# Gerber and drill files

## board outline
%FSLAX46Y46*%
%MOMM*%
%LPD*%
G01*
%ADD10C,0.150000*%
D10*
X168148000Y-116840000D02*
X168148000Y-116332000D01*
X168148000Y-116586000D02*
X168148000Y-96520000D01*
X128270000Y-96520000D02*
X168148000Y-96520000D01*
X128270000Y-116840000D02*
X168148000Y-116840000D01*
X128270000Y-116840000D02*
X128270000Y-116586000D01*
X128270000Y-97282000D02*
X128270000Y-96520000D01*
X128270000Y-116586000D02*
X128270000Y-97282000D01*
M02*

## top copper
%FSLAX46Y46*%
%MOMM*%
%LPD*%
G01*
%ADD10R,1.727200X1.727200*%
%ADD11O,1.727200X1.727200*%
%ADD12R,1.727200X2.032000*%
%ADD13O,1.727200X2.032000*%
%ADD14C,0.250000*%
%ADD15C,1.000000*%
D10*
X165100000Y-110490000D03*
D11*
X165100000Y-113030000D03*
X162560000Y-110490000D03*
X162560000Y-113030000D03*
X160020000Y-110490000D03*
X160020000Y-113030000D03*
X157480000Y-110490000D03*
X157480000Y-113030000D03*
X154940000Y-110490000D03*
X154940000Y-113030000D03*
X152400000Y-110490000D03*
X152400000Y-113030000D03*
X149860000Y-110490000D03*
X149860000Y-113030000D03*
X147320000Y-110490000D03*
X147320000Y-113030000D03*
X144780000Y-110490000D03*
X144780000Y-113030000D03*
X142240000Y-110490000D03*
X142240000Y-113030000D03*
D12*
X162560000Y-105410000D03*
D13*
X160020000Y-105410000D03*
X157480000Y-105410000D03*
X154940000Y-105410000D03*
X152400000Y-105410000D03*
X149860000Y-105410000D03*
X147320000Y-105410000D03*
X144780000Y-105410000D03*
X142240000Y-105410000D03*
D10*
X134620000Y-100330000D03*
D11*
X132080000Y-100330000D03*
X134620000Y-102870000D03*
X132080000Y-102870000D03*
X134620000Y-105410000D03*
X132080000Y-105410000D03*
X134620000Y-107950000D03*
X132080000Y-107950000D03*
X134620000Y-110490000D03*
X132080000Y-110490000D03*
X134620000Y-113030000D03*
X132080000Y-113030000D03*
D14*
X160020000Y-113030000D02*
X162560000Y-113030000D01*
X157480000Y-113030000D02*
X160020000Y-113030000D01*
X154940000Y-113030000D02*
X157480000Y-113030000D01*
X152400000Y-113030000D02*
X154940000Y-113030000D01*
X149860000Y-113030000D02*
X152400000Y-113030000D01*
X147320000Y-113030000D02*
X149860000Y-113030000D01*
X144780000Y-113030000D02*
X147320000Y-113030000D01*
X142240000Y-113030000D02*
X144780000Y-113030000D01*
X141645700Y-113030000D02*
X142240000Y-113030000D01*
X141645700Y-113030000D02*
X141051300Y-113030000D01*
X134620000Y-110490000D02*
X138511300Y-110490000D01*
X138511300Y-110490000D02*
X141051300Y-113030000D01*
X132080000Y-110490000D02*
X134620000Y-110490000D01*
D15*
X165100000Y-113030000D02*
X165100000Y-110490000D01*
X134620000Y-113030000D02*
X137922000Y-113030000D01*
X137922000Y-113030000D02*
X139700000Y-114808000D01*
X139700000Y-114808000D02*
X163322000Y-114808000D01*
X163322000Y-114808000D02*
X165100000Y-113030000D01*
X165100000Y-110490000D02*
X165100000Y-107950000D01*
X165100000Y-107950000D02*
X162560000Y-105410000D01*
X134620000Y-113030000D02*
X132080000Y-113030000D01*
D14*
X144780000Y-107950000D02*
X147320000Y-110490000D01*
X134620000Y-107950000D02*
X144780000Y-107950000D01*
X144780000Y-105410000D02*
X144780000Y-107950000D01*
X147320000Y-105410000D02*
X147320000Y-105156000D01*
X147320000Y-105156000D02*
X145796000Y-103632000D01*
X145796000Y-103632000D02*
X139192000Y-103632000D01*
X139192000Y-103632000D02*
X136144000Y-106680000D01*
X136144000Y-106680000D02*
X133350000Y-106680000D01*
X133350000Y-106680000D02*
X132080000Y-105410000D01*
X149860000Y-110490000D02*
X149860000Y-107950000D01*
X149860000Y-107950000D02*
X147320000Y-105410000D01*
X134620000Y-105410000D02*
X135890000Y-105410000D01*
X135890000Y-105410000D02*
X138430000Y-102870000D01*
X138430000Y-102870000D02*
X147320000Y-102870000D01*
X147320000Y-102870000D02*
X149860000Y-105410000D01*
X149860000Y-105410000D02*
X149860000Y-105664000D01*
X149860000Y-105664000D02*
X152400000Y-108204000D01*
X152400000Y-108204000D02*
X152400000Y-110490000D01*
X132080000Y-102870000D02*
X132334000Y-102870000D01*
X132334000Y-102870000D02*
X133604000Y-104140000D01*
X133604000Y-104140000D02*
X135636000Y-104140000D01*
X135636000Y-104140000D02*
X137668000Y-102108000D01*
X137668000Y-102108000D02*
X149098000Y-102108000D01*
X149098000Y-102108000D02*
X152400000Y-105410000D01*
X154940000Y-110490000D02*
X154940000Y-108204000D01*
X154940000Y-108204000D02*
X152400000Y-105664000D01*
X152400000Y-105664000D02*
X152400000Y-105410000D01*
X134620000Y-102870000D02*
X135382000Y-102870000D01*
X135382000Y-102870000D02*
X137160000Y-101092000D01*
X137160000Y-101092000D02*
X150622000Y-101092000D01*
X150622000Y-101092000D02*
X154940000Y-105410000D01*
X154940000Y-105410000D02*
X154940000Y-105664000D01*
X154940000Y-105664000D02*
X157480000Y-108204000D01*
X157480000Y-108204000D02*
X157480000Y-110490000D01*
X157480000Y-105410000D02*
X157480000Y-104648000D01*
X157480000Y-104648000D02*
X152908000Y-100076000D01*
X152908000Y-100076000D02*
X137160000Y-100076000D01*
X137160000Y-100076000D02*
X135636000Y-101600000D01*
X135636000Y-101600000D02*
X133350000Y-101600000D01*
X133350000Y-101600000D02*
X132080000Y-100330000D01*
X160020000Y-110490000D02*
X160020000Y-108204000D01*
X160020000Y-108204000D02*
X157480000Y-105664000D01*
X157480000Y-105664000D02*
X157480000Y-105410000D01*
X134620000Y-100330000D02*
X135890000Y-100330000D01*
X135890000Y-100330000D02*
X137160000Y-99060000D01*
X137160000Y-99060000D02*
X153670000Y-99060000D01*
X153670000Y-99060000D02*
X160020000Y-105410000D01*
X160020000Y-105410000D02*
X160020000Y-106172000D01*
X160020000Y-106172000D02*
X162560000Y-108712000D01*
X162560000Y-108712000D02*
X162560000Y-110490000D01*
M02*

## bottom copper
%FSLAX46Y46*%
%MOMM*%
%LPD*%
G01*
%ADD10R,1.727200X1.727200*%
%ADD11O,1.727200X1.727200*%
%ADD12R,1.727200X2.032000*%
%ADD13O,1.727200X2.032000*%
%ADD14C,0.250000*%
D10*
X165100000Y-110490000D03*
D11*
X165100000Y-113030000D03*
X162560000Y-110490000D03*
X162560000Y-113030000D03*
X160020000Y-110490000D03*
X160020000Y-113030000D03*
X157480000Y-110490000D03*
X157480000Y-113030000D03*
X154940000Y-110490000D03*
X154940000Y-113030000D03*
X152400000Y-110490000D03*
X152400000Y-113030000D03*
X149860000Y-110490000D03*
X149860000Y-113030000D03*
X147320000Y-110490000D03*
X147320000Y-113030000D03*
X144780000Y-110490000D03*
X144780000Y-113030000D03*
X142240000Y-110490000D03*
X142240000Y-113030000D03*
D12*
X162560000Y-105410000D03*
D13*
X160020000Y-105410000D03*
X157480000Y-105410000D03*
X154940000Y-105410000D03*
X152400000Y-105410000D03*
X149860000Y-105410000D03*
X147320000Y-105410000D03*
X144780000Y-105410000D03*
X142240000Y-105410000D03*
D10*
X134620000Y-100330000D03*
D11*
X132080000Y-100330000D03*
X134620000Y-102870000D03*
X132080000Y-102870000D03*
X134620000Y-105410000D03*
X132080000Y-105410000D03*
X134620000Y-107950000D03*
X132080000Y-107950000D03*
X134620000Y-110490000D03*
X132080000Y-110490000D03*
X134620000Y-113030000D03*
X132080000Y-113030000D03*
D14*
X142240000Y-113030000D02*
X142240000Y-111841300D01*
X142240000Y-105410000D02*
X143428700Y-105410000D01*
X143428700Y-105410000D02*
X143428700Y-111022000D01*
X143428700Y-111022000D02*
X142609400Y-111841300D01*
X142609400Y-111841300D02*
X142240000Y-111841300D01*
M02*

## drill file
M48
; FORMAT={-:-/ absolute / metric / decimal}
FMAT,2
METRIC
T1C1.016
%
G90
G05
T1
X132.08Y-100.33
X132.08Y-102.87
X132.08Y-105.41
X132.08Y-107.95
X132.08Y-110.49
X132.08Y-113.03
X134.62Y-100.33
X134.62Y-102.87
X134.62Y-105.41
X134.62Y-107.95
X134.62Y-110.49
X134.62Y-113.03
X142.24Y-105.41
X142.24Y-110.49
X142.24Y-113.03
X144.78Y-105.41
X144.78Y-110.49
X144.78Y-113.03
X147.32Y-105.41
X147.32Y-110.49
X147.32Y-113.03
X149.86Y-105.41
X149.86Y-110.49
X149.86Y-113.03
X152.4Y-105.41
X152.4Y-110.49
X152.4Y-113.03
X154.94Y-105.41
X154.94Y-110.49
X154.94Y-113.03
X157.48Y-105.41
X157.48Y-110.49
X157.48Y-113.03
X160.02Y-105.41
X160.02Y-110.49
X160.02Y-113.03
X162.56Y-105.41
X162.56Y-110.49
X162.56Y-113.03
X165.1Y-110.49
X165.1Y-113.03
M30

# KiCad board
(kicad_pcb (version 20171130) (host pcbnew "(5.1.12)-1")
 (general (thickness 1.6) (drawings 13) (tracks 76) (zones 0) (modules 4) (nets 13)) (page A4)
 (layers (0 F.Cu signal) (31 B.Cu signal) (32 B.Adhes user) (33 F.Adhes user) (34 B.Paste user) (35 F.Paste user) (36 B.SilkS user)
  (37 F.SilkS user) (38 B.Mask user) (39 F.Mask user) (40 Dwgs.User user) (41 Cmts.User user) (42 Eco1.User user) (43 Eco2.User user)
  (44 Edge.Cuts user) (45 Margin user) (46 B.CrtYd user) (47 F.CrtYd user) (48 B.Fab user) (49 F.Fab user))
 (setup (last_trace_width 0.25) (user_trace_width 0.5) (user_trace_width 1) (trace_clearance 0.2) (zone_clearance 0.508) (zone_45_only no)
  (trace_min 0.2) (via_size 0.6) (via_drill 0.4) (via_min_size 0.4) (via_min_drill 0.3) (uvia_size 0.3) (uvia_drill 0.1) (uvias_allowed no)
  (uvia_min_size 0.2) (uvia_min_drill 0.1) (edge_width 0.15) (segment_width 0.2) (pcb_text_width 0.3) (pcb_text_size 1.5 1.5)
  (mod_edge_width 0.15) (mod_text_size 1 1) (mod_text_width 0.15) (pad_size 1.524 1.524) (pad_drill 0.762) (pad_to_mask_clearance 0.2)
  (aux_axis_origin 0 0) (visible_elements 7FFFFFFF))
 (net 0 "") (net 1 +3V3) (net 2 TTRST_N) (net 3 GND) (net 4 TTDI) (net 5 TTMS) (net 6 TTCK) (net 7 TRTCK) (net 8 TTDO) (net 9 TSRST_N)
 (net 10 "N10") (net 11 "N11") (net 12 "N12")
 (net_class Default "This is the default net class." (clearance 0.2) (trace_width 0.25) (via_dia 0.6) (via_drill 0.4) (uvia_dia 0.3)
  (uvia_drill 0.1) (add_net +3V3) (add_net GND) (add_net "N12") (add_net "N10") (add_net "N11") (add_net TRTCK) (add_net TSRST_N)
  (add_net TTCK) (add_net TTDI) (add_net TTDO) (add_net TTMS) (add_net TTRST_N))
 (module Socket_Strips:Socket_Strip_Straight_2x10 (layer B.Cu) (at 165.1 110.49 180)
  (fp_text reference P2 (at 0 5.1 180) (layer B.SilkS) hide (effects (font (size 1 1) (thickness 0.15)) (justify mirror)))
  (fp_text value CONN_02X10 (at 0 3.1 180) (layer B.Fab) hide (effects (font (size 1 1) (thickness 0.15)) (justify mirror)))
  (pad 1 thru_hole rect (at 0 0 180) (size 1.7272 1.7272) (drill 1.016) (layers *.Cu *.Mask B.SilkS) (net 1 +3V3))
  (pad 2 thru_hole oval (at 0 -2.54 180) (size 1.7272 1.7272) (drill 1.016) (layers *.Cu *.Mask B.SilkS) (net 1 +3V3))
  (pad 3 thru_hole oval (at 2.54 0 180) (size 1.7272 1.7272) (drill 1.016) (layers *.Cu *.Mask B.SilkS) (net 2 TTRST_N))
  (pad 4 thru_hole oval (at 2.54 -2.54 180) (size 1.7272 1.7272) (drill 1.016) (layers *.Cu *.Mask B.SilkS) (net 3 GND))
  (pad 5 thru_hole oval (at 5.08 0 180) (size 1.7272 1.7272) (drill 1.016) (layers *.Cu *.Mask B.SilkS) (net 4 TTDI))
  (pad 6 thru_hole oval (at 5.08 -2.54 180) (size 1.7272 1.7272) (drill 1.016) (layers *.Cu *.Mask B.SilkS) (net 3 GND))
  (pad 7 thru_hole oval (at 7.62 0 180) (size 1.7272 1.7272) (drill 1.016) (layers *.Cu *.Mask B.SilkS) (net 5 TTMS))
  (pad 8 thru_hole oval (at 7.62 -2.54 180) (size 1.7272 1.7272) (drill 1.016) (layers *.Cu *.Mask B.SilkS) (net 3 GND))
  (pad 9 thru_hole oval (at 10.16 0 180) (size 1.7272 1.7272) (drill 1.016) (layers *.Cu *.Mask B.SilkS) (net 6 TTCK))
  (pad 10 thru_hole oval (at 10.16 -2.54 180) (size 1.7272 1.7272) (drill 1.016) (layers *.Cu *.Mask B.SilkS) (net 3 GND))
  (pad 11 thru_hole oval (at 12.7 0 180) (size 1.7272 1.7272) (drill 1.016) (layers *.Cu *.Mask B.SilkS) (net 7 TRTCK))
  (pad 12 thru_hole oval (at 12.7 -2.54 180) (size 1.7272 1.7272) (drill 1.016) (layers *.Cu *.Mask B.SilkS) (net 3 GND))
  (pad 13 thru_hole oval (at 15.24 0 180) (size 1.7272 1.7272) (drill 1.016) (layers *.Cu *.Mask B.SilkS) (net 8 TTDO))
  (pad 14 thru_hole oval (at 15.24 -2.54 180) (size 1.7272 1.7272) (drill 1.016) (layers *.Cu *.Mask B.SilkS) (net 3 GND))
  (pad 15 thru_hole oval (at 17.78 0 180) (size 1.7272 1.7272) (drill 1.016) (layers *.Cu *.Mask B.SilkS) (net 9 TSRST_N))
  (pad 16 thru_hole oval (at 17.78 -2.54 180) (size 1.7272 1.7272) (drill 1.016) (layers *.Cu *.Mask B.SilkS) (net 3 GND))
  (pad 17 thru_hole oval (at 20.32 0 180) (size 1.7272 1.7272) (drill 1.016) (layers *.Cu *.Mask B.SilkS) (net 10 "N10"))
  (pad 18 thru_hole oval (at 20.32 -2.54 180) (size 1.7272 1.7272) (drill 1.016) (layers *.Cu *.Mask B.SilkS) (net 3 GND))
  (pad 19 thru_hole oval (at 22.86 0 180) (size 1.7272 1.7272) (drill 1.016) (layers *.Cu *.Mask B.SilkS) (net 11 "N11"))
  (pad 20 thru_hole oval (at 22.86 -2.54 180) (size 1.7272 1.7272) (drill 1.016) (layers *.Cu *.Mask B.SilkS) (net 3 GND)))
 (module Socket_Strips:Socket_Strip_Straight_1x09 (layer F.Cu) (at 162.56 105.41 180)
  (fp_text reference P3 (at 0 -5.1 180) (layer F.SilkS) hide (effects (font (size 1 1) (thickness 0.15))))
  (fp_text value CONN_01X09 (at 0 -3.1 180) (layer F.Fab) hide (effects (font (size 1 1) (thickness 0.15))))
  (pad 1 thru_hole rect (at 0 0 180) (size 1.7272 2.032) (drill 1.016) (layers *.Cu *.Mask F.SilkS) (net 1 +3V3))
  (pad 2 thru_hole oval (at 2.54 0 180) (size 1.7272 2.032) (drill 1.016) (layers *.Cu *.Mask F.SilkS) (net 2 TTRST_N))
  (pad 3 thru_hole oval (at 5.08 0 180) (size 1.7272 2.032) (drill 1.016) (layers *.Cu *.Mask F.SilkS) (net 4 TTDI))
  (pad 4 thru_hole oval (at 7.62 0 180) (size 1.7272 2.032) (drill 1.016) (layers *.Cu *.Mask F.SilkS) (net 5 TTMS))
  (pad 5 thru_hole oval (at 10.16 0 180) (size 1.7272 2.032) (drill 1.016) (layers *.Cu *.Mask F.SilkS) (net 6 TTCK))
  (pad 6 thru_hole oval (at 12.7 0 180) (size 1.7272 2.032) (drill 1.016) (layers *.Cu *.Mask F.SilkS) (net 7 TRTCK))
  (pad 7 thru_hole oval (at 15.24 0 180) (size 1.7272 2.032) (drill 1.016) (layers *.Cu *.Mask F.SilkS) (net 8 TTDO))
  (pad 8 thru_hole oval (at 17.78 0 180) (size 1.7272 2.032) (drill 1.016) (layers *.Cu *.Mask F.SilkS) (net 9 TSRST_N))
  (pad 9 thru_hole oval (at 20.32 0 180) (size 1.7272 2.032) (drill 1.016) (layers *.Cu *.Mask F.SilkS) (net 3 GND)))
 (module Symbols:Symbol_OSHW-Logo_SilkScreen (layer B.Cu) (at 139.7 99.568 180)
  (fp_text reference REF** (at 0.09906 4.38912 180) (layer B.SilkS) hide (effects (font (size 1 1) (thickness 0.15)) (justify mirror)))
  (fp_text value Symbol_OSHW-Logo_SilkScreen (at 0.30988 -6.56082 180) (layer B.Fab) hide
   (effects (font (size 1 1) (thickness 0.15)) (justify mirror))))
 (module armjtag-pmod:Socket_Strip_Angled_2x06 (layer F.Cu) (at 134.62 100.33 270)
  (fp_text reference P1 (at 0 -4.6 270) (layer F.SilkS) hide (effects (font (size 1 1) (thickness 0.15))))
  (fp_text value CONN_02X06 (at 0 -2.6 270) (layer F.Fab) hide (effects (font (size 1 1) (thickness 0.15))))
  (pad 1 thru_hole rect (at 0 0 270) (size 1.7272 1.7272) (drill 1.016) (layers *.Cu *.Mask F.SilkS) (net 2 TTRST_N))
  (pad 2 thru_hole oval (at 0 2.54 270) (size 1.7272 1.7272) (drill 1.016) (layers *.Cu *.Mask F.SilkS) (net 4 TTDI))
  (pad 3 thru_hole oval (at 2.54 0 270) (size 1.7272 1.7272) (drill 1.016) (layers *.Cu *.Mask F.SilkS) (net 5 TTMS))
  (pad 4 thru_hole oval (at 2.54 2.54 270) (size 1.7272 1.7272) (drill 1.016) (layers *.Cu *.Mask F.SilkS) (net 6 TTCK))
  (pad 5 thru_hole oval (at 5.08 0 270) (size 1.7272 1.7272) (drill 1.016) (layers *.Cu *.Mask F.SilkS) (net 7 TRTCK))
  (pad 6 thru_hole oval (at 5.08 2.54 270) (size 1.7272 1.7272) (drill 1.016) (layers *.Cu *.Mask F.SilkS) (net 8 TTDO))
  (pad 7 thru_hole oval (at 7.62 0 270) (size 1.7272 1.7272) (drill 1.016) (layers *.Cu *.Mask F.SilkS) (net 9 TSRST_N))
  (pad 8 thru_hole oval (at 7.62 2.54 270) (size 1.7272 1.7272) (drill 1.016) (layers *.Cu *.Mask F.SilkS) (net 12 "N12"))
  (pad 9 thru_hole oval (at 10.16 0 270) (size 1.7272 1.7272) (drill 1.016) (layers *.Cu *.Mask F.SilkS) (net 3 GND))
  (pad 10 thru_hole oval (at 10.16 2.54 270) (size 1.7272 1.7272) (drill 1.016) (layers *.Cu *.Mask F.SilkS) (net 3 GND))
  (pad 11 thru_hole oval (at 12.7 0 270) (size 1.7272 1.7272) (drill 1.016) (layers *.Cu *.Mask F.SilkS) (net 1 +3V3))
  (pad 12 thru_hole oval (at 12.7 2.54 270) (size 1.7272 1.7272) (drill 1.016) (layers *.Cu *.Mask F.SilkS) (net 1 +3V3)))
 (gr_line (start 168.148 116.84) (end 168.148 116.332) (angle 90) (layer Edge.Cuts) (width 0.15))
 (gr_line (start 168.148 116.586) (end 168.148 96.52) (angle 90) (layer Edge.Cuts) (width 0.15))
 (gr_line (start 128.27 96.52) (end 168.148 96.52) (angle 90) (layer Edge.Cuts) (width 0.15))
 (gr_line (start 128.27 116.84) (end 168.148 116.84) (angle 90) (layer Edge.Cuts) (width 0.15))
 (gr_line (start 128.27 116.84) (end 128.27 116.586) (angle 90) (layer Edge.Cuts) (width 0.15))
 (gr_line (start 128.27 97.282) (end 128.27 96.52) (angle 90) (layer Edge.Cuts) (width 0.15))
 (gr_line (start 128.27 116.586) (end 128.27 97.282) (angle 90) (layer Edge.Cuts) (width 0.15))
 (segment (start 160.02 113.03) (end 162.56 113.03) (width 0.25) (layer F.Cu) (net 3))
 (segment (start 157.48 113.03) (end 160.02 113.03) (width 0.25) (layer F.Cu) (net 3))
 (segment (start 154.94 113.03) (end 157.48 113.03) (width 0.25) (layer F.Cu) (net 3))
 (segment (start 152.4 113.03) (end 154.94 113.03) (width 0.25) (layer F.Cu) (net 3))
 (segment (start 149.86 113.03) (end 152.4 113.03) (width 0.25) (layer F.Cu) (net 3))
 (segment (start 147.32 113.03) (end 149.86 113.03) (width 0.25) (layer F.Cu) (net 3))
 (segment (start 144.78 113.03) (end 147.32 113.03) (width 0.25) (layer F.Cu) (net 3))
 (segment (start 142.24 113.03) (end 144.78 113.03) (width 0.25) (layer F.Cu) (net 3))
 (segment (start 141.6457 113.03) (end 142.24 113.03) (width 0.25) (layer F.Cu) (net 3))
 (segment (start 141.6457 113.03) (end 141.0513 113.03) (width 0.25) (layer F.Cu) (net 3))
 (segment (start 142.24 113.03) (end 142.24 111.8413) (width 0.25) (layer B.Cu) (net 3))
 (segment (start 142.24 105.41) (end 143.4287 105.41) (width 0.25) (layer B.Cu) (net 3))
 (segment (start 143.4287 105.41) (end 143.4287 111.022) (width 0.25) (layer B.Cu) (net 3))
 (segment (start 143.4287 111.022) (end 142.6094 111.8413) (width 0.25) (layer B.Cu) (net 3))
 (segment (start 142.6094 111.8413) (end 142.24 111.8413) (width 0.25) (layer B.Cu) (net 3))
 (segment (start 134.62 110.49) (end 138.5113 110.49) (width 0.25) (layer F.Cu) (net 3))
 (segment (start 138.5113 110.49) (end 141.0513 113.03) (width 0.25) (layer F.Cu) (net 3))
 (segment (start 132.08 110.49) (end 134.62 110.49) (width 0.25) (layer F.Cu) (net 3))
 (segment (start 165.1 113.03) (end 165.1 110.49) (width 1) (layer F.Cu) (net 1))
 (segment (start 134.62 113.03) (end 137.922 113.03) (width 1) (layer F.Cu) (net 1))
 (segment (start 137.922 113.03) (end 139.7 114.808) (width 1) (layer F.Cu) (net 1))
 (segment (start 139.7 114.808) (end 163.322 114.808) (width 1) (layer F.Cu) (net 1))
 (segment (start 163.322 114.808) (end 165.1 113.03) (width 1) (layer F.Cu) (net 1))
 (segment (start 165.1 110.49) (end 165.1 107.95) (width 1) (layer F.Cu) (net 1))
 (segment (start 165.1 107.95) (end 162.56 105.41) (width 1) (layer F.Cu) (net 1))
 (segment (start 134.62 113.03) (end 132.08 113.03) (width 1) (layer F.Cu) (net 1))
 (segment (start 144.78 107.95) (end 147.32 110.49) (width 0.25) (layer F.Cu) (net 9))
 (segment (start 134.62 107.95) (end 144.78 107.95) (width 0.25) (layer F.Cu) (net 9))
 (segment (start 144.78 105.41) (end 144.78 107.95) (width 0.25) (layer F.Cu) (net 9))
 (segment (start 147.32 105.41) (end 147.32 105.156) (width 0.25) (layer F.Cu) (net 8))
 (segment (start 147.32 105.156) (end 145.796 103.632) (width 0.25) (layer F.Cu) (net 8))
 (segment (start 145.796 103.632) (end 139.192 103.632) (width 0.25) (layer F.Cu) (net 8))
 (segment (start 139.192 103.632) (end 136.144 106.68) (width 0.25) (layer F.Cu) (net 8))
 (segment (start 136.144 106.68) (end 133.35 106.68) (width 0.25) (layer F.Cu) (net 8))
 (segment (start 133.35 106.68) (end 132.08 105.41) (width 0.25) (layer F.Cu) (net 8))
 (segment (start 149.86 110.49) (end 149.86 107.95) (width 0.25) (layer F.Cu) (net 8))
 (segment (start 149.86 107.95) (end 147.32 105.41) (width 0.25) (layer F.Cu) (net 8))
 (segment (start 134.62 105.41) (end 135.89 105.41) (width 0.25) (layer F.Cu) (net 7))
 (segment (start 135.89 105.41) (end 138.43 102.87) (width 0.25) (layer F.Cu) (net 7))
 (segment (start 138.43 102.87) (end 147.32 102.87) (width 0.25) (layer F.Cu) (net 7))
 (segment (start 147.32 102.87) (end 149.86 105.41) (width 0.25) (layer F.Cu) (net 7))
 (segment (start 149.86 105.41) (end 149.86 105.664) (width 0.25) (layer F.Cu) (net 7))
 (segment (start 149.86 105.664) (end 152.4 108.204) (width 0.25) (layer F.Cu) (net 7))
 (segment (start 152.4 108.204) (end 152.4 110.49) (width 0.25) (layer F.Cu) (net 7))
 (segment (start 132.08 102.87) (end 132.334 102.87) (width 0.25) (layer F.Cu) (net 6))
 (segment (start 132.334 102.87) (end 133.604 104.14) (width 0.25) (layer F.Cu) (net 6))
 (segment (start 133.604 104.14) (end 135.636 104.14) (width 0.25) (layer F.Cu) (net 6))
 (segment (start 135.636 104.14) (end 137.668 102.108) (width 0.25) (layer F.Cu) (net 6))
 (segment (start 137.668 102.108) (end 149.098 102.108) (width 0.25) (layer F.Cu) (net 6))
 (segment (start 149.098 102.108) (end 152.4 105.41) (width 0.25) (layer F.Cu) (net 6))
 (segment (start 154.94 110.49) (end 154.94 108.204) (width 0.25) (layer F.Cu) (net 6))
 (segment (start 154.94 108.204) (end 152.4 105.664) (width 0.25) (layer F.Cu) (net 6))
 (segment (start 152.4 105.664) (end 152.4 105.41) (width 0.25) (layer F.Cu) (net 6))
 (segment (start 134.62 102.87) (end 135.382 102.87) (width 0.25) (layer F.Cu) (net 5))
 (segment (start 135.382 102.87) (end 137.16 101.092) (width 0.25) (layer F.Cu) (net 5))
 (segment (start 137.16 101.092) (end 150.622 101.092) (width 0.25) (layer F.Cu) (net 5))
 (segment (start 150.622 101.092) (end 154.94 105.41) (width 0.25) (layer F.Cu) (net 5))
 (segment (start 154.94 105.41) (end 154.94 105.664) (width 0.25) (layer F.Cu) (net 5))
 (segment (start 154.94 105.664) (end 157.48 108.204) (width 0.25) (layer F.Cu) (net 5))
 (segment (start 157.48 108.204) (end 157.48 110.49) (width 0.25) (layer F.Cu) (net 5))
 (segment (start 157.48 105.41) (end 157.48 104.648) (width 0.25) (layer F.Cu) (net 4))
 (segment (start 157.48 104.648) (end 152.908 100.076) (width 0.25) (layer F.Cu) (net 4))
 (segment (start 152.908 100.076) (end 137.16 100.076) (width 0.25) (layer F.Cu) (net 4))
 (segment (start 137.16 100.076) (end 135.636 101.6) (width 0.25) (layer F.Cu) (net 4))
 (segment (start 135.636 101.6) (end 133.35 101.6) (width 0.25) (layer F.Cu) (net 4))
 (segment (start 133.35 101.6) (end 132.08 100.33) (width 0.25) (layer F.Cu) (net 4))
 (segment (start 160.02 110.49) (end 160.02 108.204) (width 0.25) (layer F.Cu) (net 4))
 (segment (start 160.02 108.204) (end 157.48 105.664) (width 0.25) (layer F.Cu) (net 4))
 (segment (start 157.48 105.664) (end 157.48 105.41) (width 0.25) (layer F.Cu) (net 4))
 (segment (start 134.62 100.33) (end 135.89 100.33) (width 0.25) (layer F.Cu) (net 2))
 (segment (start 135.89 100.33) (end 137.16 99.06) (width 0.25) (layer F.Cu) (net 2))
 (segment (start 137.16 99.06) (end 153.67 99.06) (width 0.25) (layer F.Cu) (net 2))
 (segment (start 153.67 99.06) (end 160.02 105.41) (width 0.25) (layer F.Cu) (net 2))
 (segment (start 160.02 105.41) (end 160.02 106.172) (width 0.25) (layer F.Cu) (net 2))
 (segment (start 160.02 106.172) (end 162.56 108.712) (width 0.25) (layer F.Cu) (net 2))
 (segment (start 162.56 108.712) (end 162.56 110.49) (width 0.25) (layer F.Cu) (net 2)))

